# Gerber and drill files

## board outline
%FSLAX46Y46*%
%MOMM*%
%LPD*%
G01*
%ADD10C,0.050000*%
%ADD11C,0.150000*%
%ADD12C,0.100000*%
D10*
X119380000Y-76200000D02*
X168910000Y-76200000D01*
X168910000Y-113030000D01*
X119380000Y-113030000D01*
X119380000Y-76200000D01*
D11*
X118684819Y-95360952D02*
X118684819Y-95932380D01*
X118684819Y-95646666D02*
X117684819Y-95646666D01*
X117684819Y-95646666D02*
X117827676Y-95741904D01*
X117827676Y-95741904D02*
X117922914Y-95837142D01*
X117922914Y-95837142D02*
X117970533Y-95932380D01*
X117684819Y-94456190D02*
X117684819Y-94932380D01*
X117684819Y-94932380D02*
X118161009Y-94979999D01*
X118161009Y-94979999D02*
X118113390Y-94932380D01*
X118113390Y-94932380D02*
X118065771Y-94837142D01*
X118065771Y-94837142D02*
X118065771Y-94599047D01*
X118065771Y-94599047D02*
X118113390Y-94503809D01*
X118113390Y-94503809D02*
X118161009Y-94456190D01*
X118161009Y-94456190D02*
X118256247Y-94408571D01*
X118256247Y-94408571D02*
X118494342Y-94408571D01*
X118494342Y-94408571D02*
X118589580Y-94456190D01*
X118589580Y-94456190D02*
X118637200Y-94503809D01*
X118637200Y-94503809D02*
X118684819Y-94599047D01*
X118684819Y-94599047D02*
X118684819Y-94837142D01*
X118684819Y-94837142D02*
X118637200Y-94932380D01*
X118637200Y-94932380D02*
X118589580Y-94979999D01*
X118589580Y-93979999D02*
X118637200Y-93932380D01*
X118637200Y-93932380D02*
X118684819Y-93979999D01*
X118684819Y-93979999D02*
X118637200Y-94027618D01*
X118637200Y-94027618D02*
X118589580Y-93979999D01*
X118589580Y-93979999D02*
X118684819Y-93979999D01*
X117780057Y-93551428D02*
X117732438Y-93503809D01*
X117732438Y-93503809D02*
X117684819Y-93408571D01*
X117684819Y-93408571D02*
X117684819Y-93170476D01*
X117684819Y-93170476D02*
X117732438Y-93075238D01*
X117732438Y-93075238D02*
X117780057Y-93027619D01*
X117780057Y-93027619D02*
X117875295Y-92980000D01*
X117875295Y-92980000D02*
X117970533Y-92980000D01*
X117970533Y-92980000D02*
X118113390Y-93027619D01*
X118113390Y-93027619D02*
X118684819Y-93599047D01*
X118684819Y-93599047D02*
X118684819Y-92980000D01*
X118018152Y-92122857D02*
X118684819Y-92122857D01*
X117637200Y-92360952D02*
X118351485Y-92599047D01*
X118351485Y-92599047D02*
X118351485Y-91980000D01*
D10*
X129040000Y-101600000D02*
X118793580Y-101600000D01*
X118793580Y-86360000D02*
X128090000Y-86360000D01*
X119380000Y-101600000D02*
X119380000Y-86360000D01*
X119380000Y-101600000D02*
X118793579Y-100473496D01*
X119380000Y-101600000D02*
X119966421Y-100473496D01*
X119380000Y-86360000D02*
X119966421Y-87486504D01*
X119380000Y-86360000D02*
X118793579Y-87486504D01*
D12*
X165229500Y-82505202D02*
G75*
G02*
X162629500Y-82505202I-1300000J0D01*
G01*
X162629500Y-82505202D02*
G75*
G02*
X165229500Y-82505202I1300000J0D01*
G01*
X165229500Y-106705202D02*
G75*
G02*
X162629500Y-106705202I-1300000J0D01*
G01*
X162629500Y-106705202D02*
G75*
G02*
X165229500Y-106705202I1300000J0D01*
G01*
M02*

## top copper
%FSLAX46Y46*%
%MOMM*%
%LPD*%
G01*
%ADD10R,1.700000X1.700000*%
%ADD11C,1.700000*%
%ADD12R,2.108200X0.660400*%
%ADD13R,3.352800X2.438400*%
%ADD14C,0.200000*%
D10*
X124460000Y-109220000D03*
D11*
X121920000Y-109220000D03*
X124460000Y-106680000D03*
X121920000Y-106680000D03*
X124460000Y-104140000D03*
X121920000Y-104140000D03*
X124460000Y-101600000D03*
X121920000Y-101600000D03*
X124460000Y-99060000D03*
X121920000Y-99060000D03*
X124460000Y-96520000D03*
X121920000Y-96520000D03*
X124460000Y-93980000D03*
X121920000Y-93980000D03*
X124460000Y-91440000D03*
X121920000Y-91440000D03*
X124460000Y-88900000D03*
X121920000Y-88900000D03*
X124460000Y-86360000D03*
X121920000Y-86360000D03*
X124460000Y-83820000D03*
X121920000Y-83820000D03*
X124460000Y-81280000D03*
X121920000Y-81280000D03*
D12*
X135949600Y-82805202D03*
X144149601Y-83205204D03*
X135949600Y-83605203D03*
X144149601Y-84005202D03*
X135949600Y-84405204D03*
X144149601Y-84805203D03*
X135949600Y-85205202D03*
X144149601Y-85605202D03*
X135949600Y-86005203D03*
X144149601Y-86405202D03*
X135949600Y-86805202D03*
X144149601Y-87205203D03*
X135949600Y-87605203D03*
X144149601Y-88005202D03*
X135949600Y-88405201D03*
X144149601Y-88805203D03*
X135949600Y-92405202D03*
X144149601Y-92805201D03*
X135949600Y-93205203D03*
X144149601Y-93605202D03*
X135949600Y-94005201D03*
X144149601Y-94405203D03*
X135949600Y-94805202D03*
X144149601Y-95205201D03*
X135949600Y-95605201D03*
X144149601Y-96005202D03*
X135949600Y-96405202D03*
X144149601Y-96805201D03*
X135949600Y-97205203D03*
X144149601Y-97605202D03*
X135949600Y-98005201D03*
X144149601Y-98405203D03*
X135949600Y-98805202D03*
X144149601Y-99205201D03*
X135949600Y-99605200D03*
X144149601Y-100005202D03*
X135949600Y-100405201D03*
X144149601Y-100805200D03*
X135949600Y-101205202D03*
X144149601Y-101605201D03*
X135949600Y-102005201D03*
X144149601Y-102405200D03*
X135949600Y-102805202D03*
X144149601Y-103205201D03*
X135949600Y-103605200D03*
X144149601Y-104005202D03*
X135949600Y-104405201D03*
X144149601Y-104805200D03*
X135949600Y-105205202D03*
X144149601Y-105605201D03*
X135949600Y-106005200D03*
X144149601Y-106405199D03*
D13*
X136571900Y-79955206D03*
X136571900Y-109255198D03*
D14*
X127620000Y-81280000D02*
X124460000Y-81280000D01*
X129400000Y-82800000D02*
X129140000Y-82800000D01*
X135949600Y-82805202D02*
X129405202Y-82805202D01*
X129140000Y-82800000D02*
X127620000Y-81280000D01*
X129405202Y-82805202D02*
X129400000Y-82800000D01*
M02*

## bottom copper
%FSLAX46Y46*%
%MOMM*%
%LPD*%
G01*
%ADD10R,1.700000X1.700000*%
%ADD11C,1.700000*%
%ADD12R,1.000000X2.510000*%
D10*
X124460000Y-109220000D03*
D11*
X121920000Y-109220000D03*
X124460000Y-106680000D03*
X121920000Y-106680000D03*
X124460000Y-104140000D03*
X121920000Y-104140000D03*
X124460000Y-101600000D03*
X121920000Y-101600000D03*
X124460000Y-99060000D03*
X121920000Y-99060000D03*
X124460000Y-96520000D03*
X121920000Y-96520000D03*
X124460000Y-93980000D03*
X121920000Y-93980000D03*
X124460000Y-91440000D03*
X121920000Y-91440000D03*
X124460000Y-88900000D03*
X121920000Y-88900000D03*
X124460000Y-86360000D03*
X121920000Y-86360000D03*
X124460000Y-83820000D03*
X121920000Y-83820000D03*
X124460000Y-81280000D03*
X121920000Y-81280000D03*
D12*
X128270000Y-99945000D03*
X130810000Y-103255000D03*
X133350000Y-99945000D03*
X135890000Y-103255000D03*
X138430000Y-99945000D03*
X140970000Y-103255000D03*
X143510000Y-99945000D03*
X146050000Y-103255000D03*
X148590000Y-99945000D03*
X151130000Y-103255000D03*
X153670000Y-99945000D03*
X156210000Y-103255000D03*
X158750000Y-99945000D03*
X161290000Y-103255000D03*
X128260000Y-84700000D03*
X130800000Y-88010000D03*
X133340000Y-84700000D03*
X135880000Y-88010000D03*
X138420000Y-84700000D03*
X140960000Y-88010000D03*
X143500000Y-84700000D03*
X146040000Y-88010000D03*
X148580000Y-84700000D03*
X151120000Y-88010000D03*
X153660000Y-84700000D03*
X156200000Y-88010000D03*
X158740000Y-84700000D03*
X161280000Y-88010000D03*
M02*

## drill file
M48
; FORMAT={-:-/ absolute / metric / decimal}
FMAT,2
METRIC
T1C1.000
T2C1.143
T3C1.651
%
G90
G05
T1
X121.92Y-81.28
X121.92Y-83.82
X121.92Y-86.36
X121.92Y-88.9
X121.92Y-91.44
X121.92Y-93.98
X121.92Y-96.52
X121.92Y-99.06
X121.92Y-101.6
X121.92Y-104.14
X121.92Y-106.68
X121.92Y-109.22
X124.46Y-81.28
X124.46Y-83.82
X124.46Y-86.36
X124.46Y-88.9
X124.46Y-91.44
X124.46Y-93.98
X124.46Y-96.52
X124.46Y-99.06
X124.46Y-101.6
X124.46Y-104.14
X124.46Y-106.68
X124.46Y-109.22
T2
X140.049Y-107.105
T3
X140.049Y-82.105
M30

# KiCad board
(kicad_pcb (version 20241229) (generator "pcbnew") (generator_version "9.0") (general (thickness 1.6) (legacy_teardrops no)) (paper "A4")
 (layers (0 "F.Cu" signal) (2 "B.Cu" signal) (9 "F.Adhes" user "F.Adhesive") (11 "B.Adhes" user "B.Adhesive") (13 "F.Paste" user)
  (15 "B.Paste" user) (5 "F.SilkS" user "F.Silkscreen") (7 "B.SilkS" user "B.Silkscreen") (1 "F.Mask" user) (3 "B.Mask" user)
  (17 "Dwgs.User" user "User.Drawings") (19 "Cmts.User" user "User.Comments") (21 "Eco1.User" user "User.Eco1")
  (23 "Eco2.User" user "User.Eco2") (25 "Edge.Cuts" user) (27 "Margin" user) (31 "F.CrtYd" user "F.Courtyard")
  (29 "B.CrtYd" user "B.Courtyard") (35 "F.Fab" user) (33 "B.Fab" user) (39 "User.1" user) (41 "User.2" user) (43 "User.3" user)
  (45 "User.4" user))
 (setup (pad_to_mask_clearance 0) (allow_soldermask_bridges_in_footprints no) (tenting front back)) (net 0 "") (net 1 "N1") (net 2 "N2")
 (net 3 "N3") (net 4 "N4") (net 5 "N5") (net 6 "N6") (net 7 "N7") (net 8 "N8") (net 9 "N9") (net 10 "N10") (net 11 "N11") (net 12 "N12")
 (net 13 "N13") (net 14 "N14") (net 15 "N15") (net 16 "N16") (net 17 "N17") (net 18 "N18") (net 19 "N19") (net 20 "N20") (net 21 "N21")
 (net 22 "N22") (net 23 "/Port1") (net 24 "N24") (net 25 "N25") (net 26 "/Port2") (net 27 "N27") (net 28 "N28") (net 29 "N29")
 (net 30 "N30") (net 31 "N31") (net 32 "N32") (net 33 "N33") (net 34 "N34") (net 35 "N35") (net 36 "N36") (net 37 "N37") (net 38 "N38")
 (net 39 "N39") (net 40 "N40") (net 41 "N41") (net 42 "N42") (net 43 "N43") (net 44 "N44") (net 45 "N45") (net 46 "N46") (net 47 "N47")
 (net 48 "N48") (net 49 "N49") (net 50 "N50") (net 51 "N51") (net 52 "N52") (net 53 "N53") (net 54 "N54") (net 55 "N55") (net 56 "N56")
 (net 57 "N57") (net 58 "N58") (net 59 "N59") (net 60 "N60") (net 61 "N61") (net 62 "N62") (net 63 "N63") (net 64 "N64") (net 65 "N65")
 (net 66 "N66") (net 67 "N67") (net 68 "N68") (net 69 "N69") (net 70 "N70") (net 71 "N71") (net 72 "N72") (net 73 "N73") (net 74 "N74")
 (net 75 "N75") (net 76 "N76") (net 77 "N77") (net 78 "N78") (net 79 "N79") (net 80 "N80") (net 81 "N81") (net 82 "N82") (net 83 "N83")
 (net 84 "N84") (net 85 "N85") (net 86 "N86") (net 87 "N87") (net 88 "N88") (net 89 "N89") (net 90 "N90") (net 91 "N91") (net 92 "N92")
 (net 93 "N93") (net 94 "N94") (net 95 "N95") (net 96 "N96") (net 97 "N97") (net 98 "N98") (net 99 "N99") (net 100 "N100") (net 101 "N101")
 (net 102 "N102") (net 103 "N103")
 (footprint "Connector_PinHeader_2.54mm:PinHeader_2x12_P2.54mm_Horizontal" (layer "F.Cu") (at 124.46 109.22 180)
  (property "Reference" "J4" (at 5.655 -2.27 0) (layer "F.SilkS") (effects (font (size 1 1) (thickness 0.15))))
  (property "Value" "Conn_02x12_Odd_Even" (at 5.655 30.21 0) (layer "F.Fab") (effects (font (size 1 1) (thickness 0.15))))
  (pad "1" thru_hole rect (at 0 0 180) (size 1.7 1.7) (drill 1) (layers "*.Cu" "*.Mask") (remove_unused_layers no) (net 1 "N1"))
  (pad "2" thru_hole circle (at 2.54 0 180) (size 1.7 1.7) (drill 1) (layers "*.Cu" "*.Mask") (remove_unused_layers no) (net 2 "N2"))
  (pad "3" thru_hole circle (at 0 2.54 180) (size 1.7 1.7) (drill 1) (layers "*.Cu" "*.Mask") (remove_unused_layers no) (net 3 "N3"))
  (pad "4" thru_hole circle (at 2.54 2.54 180) (size 1.7 1.7) (drill 1) (layers "*.Cu" "*.Mask") (remove_unused_layers no) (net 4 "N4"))
  (pad "5" thru_hole circle (at 0 5.08 180) (size 1.7 1.7) (drill 1) (layers "*.Cu" "*.Mask") (remove_unused_layers no) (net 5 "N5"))
  (pad "6" thru_hole circle (at 2.54 5.08 180) (size 1.7 1.7) (drill 1) (layers "*.Cu" "*.Mask") (remove_unused_layers no) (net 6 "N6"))
  (pad "7" thru_hole circle (at 0 7.62 180) (size 1.7 1.7) (drill 1) (layers "*.Cu" "*.Mask") (remove_unused_layers no) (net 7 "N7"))
  (pad "8" thru_hole circle (at 2.54 7.62 180) (size 1.7 1.7) (drill 1) (layers "*.Cu" "*.Mask") (remove_unused_layers no) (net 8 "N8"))
  (pad "9" thru_hole circle (at 0 10.16 180) (size 1.7 1.7) (drill 1) (layers "*.Cu" "*.Mask") (remove_unused_layers no) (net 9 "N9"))
  (pad "10" thru_hole circle (at 2.54 10.16 180) (size 1.7 1.7) (drill 1) (layers "*.Cu" "*.Mask") (remove_unused_layers no) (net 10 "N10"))
  (pad "11" thru_hole circle (at 0 12.7 180) (size 1.7 1.7) (drill 1) (layers "*.Cu" "*.Mask") (remove_unused_layers no) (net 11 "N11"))
  (pad "12" thru_hole circle (at 2.54 12.7 180) (size 1.7 1.7) (drill 1) (layers "*.Cu" "*.Mask") (remove_unused_layers no) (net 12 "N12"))
  (pad "13" thru_hole circle (at 0 15.24 180) (size 1.7 1.7) (drill 1) (layers "*.Cu" "*.Mask") (remove_unused_layers no) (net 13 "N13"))
  (pad "14" thru_hole circle (at 2.54 15.24 180) (size 1.7 1.7) (drill 1) (layers "*.Cu" "*.Mask") (remove_unused_layers no) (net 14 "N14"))
  (pad "15" thru_hole circle (at 0 17.78 180) (size 1.7 1.7) (drill 1) (layers "*.Cu" "*.Mask") (remove_unused_layers no) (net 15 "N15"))
  (pad "16" thru_hole circle (at 2.54 17.78 180) (size 1.7 1.7) (drill 1) (layers "*.Cu" "*.Mask") (remove_unused_layers no) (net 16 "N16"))
  (pad "17" thru_hole circle (at 0 20.32 180) (size 1.7 1.7) (drill 1) (layers "*.Cu" "*.Mask") (remove_unused_layers no) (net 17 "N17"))
  (pad "18" thru_hole circle (at 2.54 20.32 180) (size 1.7 1.7) (drill 1) (layers "*.Cu" "*.Mask") (remove_unused_layers no) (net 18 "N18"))
  (pad "19" thru_hole circle (at 0 22.86 180) (size 1.7 1.7) (drill 1) (layers "*.Cu" "*.Mask") (remove_unused_layers no) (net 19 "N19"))
  (pad "20" thru_hole circle (at 2.54 22.86 180) (size 1.7 1.7) (drill 1) (layers "*.Cu" "*.Mask") (remove_unused_layers no) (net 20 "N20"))
  (pad "21" thru_hole circle (at 0 25.4 180) (size 1.7 1.7) (drill 1) (layers "*.Cu" "*.Mask") (remove_unused_layers no) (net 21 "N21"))
  (pad "22" thru_hole circle (at 2.54 25.4 180) (size 1.7 1.7) (drill 1) (layers "*.Cu" "*.Mask") (remove_unused_layers no) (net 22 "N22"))
  (pad "23" thru_hole circle (at 0 27.94 180) (size 1.7 1.7) (drill 1) (layers "*.Cu" "*.Mask") (remove_unused_layers no) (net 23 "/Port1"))
  (pad "24" thru_hole circle (at 2.54 27.94 180) (size 1.7 1.7) (drill 1) (layers "*.Cu" "*.Mask") (remove_unused_layers no) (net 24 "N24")))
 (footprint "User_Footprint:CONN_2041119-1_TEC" (layer "F.Cu") (at 140.0495 94.605202 -90)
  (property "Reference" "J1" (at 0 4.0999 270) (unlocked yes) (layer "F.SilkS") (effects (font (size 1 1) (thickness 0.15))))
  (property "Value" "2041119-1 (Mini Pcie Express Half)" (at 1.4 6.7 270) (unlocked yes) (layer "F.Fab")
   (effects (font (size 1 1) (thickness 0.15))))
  (fp_circle (center -12.1 -23.88) (end -10.8 -23.88) (stroke (width 0.1) (type solid)) (fill no) (layer "Edge.Cuts"))
  (fp_circle (center 12.1 -23.88) (end 13.4 -23.88) (stroke (width 0.1) (type solid)) (fill no) (layer "Edge.Cuts"))
  (pad "" np_thru_hole circle (at -12.500102 0 270) (size 1.651 1.651) (drill 1.651) (layers))
  (pad "" np_thru_hole circle (at 12.500102 0 270) (size 1.143 1.143) (drill 1.143) (layers))
  (pad "1" smd rect (at -11.8 4.0999 270) (size 0.6604 2.1082) (layers "F.Cu" "F.Mask" "F.Paste") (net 23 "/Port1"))
  (pad "2" smd rect (at -11.399998 -4.100101 270) (size 0.6604 2.1082) (layers "F.Cu" "F.Mask" "F.Paste") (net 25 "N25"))
  (pad "3" smd rect (at -10.999999 4.0999 270) (size 0.6604 2.1082) (layers "F.Cu" "F.Mask" "F.Paste") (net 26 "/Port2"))
  (pad "4" smd rect (at -10.6 -4.100101 270) (size 0.6604 2.1082) (layers "F.Cu" "F.Mask" "F.Paste") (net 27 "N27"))
  (pad "5" smd rect (at -10.199998 4.0999 270) (size 0.6604 2.1082) (layers "F.Cu" "F.Mask" "F.Paste") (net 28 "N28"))
  (pad "6" smd rect (at -9.799999 -4.100101 270) (size 0.6604 2.1082) (layers "F.Cu" "F.Mask" "F.Paste") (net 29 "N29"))
  (pad "7" smd rect (at -9.4 4.0999 270) (size 0.6604 2.1082) (layers "F.Cu" "F.Mask" "F.Paste") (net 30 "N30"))
  (pad "8" smd rect (at -9 -4.100101 270) (size 0.6604 2.1082) (layers "F.Cu" "F.Mask" "F.Paste") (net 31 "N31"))
  (pad "9" smd rect (at -8.599999 4.0999 270) (size 0.6604 2.1082) (layers "F.Cu" "F.Mask" "F.Paste") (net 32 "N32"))
  (pad "10" smd rect (at -8.2 -4.100101 270) (size 0.6604 2.1082) (layers "F.Cu" "F.Mask" "F.Paste") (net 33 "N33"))
  (pad "11" smd rect (at -7.8 4.0999 270) (size 0.6604 2.1082) (layers "F.Cu" "F.Mask" "F.Paste") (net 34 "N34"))
  (pad "12" smd rect (at -7.399999 -4.100101 270) (size 0.6604 2.1082) (layers "F.Cu" "F.Mask" "F.Paste") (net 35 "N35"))
  (pad "13" smd rect (at -6.999999 4.0999 270) (size 0.6604 2.1082) (layers "F.Cu" "F.Mask" "F.Paste") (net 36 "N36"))
  (pad "14" smd rect (at -6.6 -4.100101 270) (size 0.6604 2.1082) (layers "F.Cu" "F.Mask" "F.Paste") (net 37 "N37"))
  (pad "15" smd rect (at -6.200001 4.0999 270) (size 0.6604 2.1082) (layers "F.Cu" "F.Mask" "F.Paste") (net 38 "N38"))
  (pad "16" smd rect (at -5.799999 -4.100101 270) (size 0.6604 2.1082) (layers "F.Cu" "F.Mask" "F.Paste") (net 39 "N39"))
  (pad "17" smd rect (at -2.2 4.0999 270) (size 0.6604 2.1082) (layers "F.Cu" "F.Mask" "F.Paste") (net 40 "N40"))
  (pad "18" smd rect (at -1.800001 -4.100101 270) (size 0.6604 2.1082) (layers "F.Cu" "F.Mask" "F.Paste") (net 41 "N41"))
  (pad "19" smd rect (at -1.399999 4.0999 270) (size 0.6604 2.1082) (layers "F.Cu" "F.Mask" "F.Paste") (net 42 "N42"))
  (pad "20" smd rect (at -1 -4.100101 270) (size 0.6604 2.1082) (layers "F.Cu" "F.Mask" "F.Paste") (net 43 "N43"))
  (pad "21" smd rect (at -0.600001 4.0999 270) (size 0.6604 2.1082) (layers "F.Cu" "F.Mask" "F.Paste") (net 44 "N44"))
  (pad "22" smd rect (at -0.199999 -4.100101 270) (size 0.6604 2.1082) (layers "F.Cu" "F.Mask" "F.Paste") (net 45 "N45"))
  (pad "23" smd rect (at 0.2 4.0999 270) (size 0.6604 2.1082) (layers "F.Cu" "F.Mask" "F.Paste") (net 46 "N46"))
  (pad "24" smd rect (at 0.599999 -4.100101 270) (size 0.6604 2.1082) (layers "F.Cu" "F.Mask" "F.Paste") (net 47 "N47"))
  (pad "25" smd rect (at 0.999999 4.0999 270) (size 0.6604 2.1082) (layers "F.Cu" "F.Mask" "F.Paste") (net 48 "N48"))
  (pad "26" smd rect (at 1.4 -4.100101 270) (size 0.6604 2.1082) (layers "F.Cu" "F.Mask" "F.Paste") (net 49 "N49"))
  (pad "27" smd rect (at 1.8 4.0999 270) (size 0.6604 2.1082) (layers "F.Cu" "F.Mask" "F.Paste") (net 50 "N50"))
  (pad "28" smd rect (at 2.199999 -4.100101 270) (size 0.6604 2.1082) (layers "F.Cu" "F.Mask" "F.Paste") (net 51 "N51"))
  (pad "29" smd rect (at 2.600001 4.0999 270) (size 0.6604 2.1082) (layers "F.Cu" "F.Mask" "F.Paste") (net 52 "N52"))
  (pad "30" smd rect (at 3 -4.100101 270) (size 0.6604 2.1082) (layers "F.Cu" "F.Mask" "F.Paste") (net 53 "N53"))
  (pad "31" smd rect (at 3.399999 4.0999 270) (size 0.6604 2.1082) (layers "F.Cu" "F.Mask" "F.Paste") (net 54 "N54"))
  (pad "32" smd rect (at 3.800001 -4.100101 270) (size 0.6604 2.1082) (layers "F.Cu" "F.Mask" "F.Paste") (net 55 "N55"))
  (pad "33" smd rect (at 4.2 4.0999 270) (size 0.6604 2.1082) (layers "F.Cu" "F.Mask" "F.Paste") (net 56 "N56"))
  (pad "34" smd rect (at 4.599999 -4.100101 270) (size 0.6604 2.1082) (layers "F.Cu" "F.Mask" "F.Paste") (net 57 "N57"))
  (pad "35" smd rect (at 4.999998 4.0999 270) (size 0.6604 2.1082) (layers "F.Cu" "F.Mask" "F.Paste") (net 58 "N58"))
  (pad "36" smd rect (at 5.4 -4.100101 270) (size 0.6604 2.1082) (layers "F.Cu" "F.Mask" "F.Paste") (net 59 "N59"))
  (pad "37" smd rect (at 5.799999 4.0999 270) (size 0.6604 2.1082) (layers "F.Cu" "F.Mask" "F.Paste") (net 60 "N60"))
  (pad "38" smd rect (at 6.199998 -4.100101 270) (size 0.6604 2.1082) (layers "F.Cu" "F.Mask" "F.Paste") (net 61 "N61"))
  (pad "39" smd rect (at 6.6 4.0999 270) (size 0.6604 2.1082) (layers "F.Cu" "F.Mask" "F.Paste") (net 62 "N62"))
  (pad "40" smd rect (at 6.999999 -4.100101 270) (size 0.6604 2.1082) (layers "F.Cu" "F.Mask" "F.Paste") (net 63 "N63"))
  (pad "41" smd rect (at 7.399999 4.0999 270) (size 0.6604 2.1082) (layers "F.Cu" "F.Mask" "F.Paste") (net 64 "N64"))
  (pad "42" smd rect (at 7.799998 -4.100101 270) (size 0.6604 2.1082) (layers "F.Cu" "F.Mask" "F.Paste") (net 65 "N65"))
  (pad "43" smd rect (at 8.2 4.0999 270) (size 0.6604 2.1082) (layers "F.Cu" "F.Mask" "F.Paste") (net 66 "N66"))
  (pad "44" smd rect (at 8.599999 -4.100101 270) (size 0.6604 2.1082) (layers "F.Cu" "F.Mask" "F.Paste") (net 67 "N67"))
  (pad "45" smd rect (at 8.999998 4.0999 270) (size 0.6604 2.1082) (layers "F.Cu" "F.Mask" "F.Paste") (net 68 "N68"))
  (pad "46" smd rect (at 9.4 -4.100101 270) (size 0.6604 2.1082) (layers "F.Cu" "F.Mask" "F.Paste") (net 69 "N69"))
  (pad "47" smd rect (at 9.799999 4.0999 270) (size 0.6604 2.1082) (layers "F.Cu" "F.Mask" "F.Paste") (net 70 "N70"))
  (pad "48" smd rect (at 10.199998 -4.100101 270) (size 0.6604 2.1082) (layers "F.Cu" "F.Mask" "F.Paste") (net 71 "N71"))
  (pad "49" smd rect (at 10.6 4.0999 270) (size 0.6604 2.1082) (layers "F.Cu" "F.Mask" "F.Paste") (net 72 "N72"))
  (pad "50" smd rect (at 10.999999 -4.100101 270) (size 0.6604 2.1082) (layers "F.Cu" "F.Mask" "F.Paste") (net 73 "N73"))
  (pad "51" smd rect (at 11.399998 4.0999 270) (size 0.6604 2.1082) (layers "F.Cu" "F.Mask" "F.Paste") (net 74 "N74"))
  (pad "52" smd rect (at 11.799997 -4.100101 270) (size 0.6604 2.1082) (layers "F.Cu" "F.Mask" "F.Paste") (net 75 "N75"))
  (pad "53" smd rect (at -14.649996 3.4776) (size 3.3528 2.4384) (layers "F.Cu" "F.Mask" "F.Paste"))
  (pad "54" smd rect (at 14.649996 3.4776) (size 3.3528 2.4384) (layers "F.Cu" "F.Mask" "F.Paste")))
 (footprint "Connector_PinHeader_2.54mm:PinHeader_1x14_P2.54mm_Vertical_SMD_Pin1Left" (layer "B.Cu") (at 144.78 101.6 -90)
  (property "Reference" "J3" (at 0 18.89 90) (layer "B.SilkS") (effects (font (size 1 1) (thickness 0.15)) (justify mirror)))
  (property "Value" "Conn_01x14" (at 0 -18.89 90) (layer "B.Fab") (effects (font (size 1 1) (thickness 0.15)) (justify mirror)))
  (pad "1" smd rect (at -1.655 16.51 270) (size 2.51 1) (layers "B.Cu" "B.Mask" "B.Paste") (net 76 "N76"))
  (pad "2" smd rect (at 1.655 13.97 270) (size 2.51 1) (layers "B.Cu" "B.Mask" "B.Paste") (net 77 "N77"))
  (pad "3" smd rect (at -1.655 11.43 270) (size 2.51 1) (layers "B.Cu" "B.Mask" "B.Paste") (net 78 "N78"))
  (pad "4" smd rect (at 1.655 8.89 270) (size 2.51 1) (layers "B.Cu" "B.Mask" "B.Paste") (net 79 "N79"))
  (pad "5" smd rect (at -1.655 6.35 270) (size 2.51 1) (layers "B.Cu" "B.Mask" "B.Paste") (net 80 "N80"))
  (pad "6" smd rect (at 1.655 3.81 270) (size 2.51 1) (layers "B.Cu" "B.Mask" "B.Paste") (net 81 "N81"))
  (pad "7" smd rect (at -1.655 1.27 270) (size 2.51 1) (layers "B.Cu" "B.Mask" "B.Paste") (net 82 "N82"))
  (pad "8" smd rect (at 1.655 -1.27 270) (size 2.51 1) (layers "B.Cu" "B.Mask" "B.Paste") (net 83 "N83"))
  (pad "9" smd rect (at -1.655 -3.81 270) (size 2.51 1) (layers "B.Cu" "B.Mask" "B.Paste") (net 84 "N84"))
  (pad "10" smd rect (at 1.655 -6.35 270) (size 2.51 1) (layers "B.Cu" "B.Mask" "B.Paste") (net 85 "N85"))
  (pad "11" smd rect (at -1.655 -8.89 270) (size 2.51 1) (layers "B.Cu" "B.Mask" "B.Paste") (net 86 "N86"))
  (pad "12" smd rect (at 1.655 -11.43 270) (size 2.51 1) (layers "B.Cu" "B.Mask" "B.Paste") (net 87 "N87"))
  (pad "13" smd rect (at -1.655 -13.97 270) (size 2.51 1) (layers "B.Cu" "B.Mask" "B.Paste") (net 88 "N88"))
  (pad "14" smd rect (at 1.655 -16.51 270) (size 2.51 1) (layers "B.Cu" "B.Mask" "B.Paste") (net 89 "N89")))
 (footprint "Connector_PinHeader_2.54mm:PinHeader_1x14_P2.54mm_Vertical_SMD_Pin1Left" (layer "B.Cu") (at 144.77 86.355 -90)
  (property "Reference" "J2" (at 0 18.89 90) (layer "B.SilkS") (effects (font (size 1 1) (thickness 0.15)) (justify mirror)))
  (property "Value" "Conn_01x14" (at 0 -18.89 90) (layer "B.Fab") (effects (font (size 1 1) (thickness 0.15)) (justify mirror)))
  (pad "1" smd rect (at -1.655 16.51 270) (size 2.51 1) (layers "B.Cu" "B.Mask" "B.Paste") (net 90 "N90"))
  (pad "2" smd rect (at 1.655 13.97 270) (size 2.51 1) (layers "B.Cu" "B.Mask" "B.Paste") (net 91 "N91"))
  (pad "3" smd rect (at -1.655 11.43 270) (size 2.51 1) (layers "B.Cu" "B.Mask" "B.Paste") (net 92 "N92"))
  (pad "4" smd rect (at 1.655 8.89 270) (size 2.51 1) (layers "B.Cu" "B.Mask" "B.Paste") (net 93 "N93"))
  (pad "5" smd rect (at -1.655 6.35 270) (size 2.51 1) (layers "B.Cu" "B.Mask" "B.Paste") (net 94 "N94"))
  (pad "6" smd rect (at 1.655 3.81 270) (size 2.51 1) (layers "B.Cu" "B.Mask" "B.Paste") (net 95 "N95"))
  (pad "7" smd rect (at -1.655 1.27 270) (size 2.51 1) (layers "B.Cu" "B.Mask" "B.Paste") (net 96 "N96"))
  (pad "8" smd rect (at 1.655 -1.27 270) (size 2.51 1) (layers "B.Cu" "B.Mask" "B.Paste") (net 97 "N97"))
  (pad "9" smd rect (at -1.655 -3.81 270) (size 2.51 1) (layers "B.Cu" "B.Mask" "B.Paste") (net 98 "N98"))
  (pad "10" smd rect (at 1.655 -6.35 270) (size 2.51 1) (layers "B.Cu" "B.Mask" "B.Paste") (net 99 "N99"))
  (pad "11" smd rect (at -1.655 -8.89 270) (size 2.51 1) (layers "B.Cu" "B.Mask" "B.Paste") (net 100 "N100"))
  (pad "12" smd rect (at 1.655 -11.43 270) (size 2.51 1) (layers "B.Cu" "B.Mask" "B.Paste") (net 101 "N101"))
  (pad "13" smd rect (at -1.655 -13.97 270) (size 2.51 1) (layers "B.Cu" "B.Mask" "B.Paste") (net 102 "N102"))
  (pad "14" smd rect (at 1.655 -16.51 270) (size 2.51 1) (layers "B.Cu" "B.Mask" "B.Paste") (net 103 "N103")))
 (gr_rect (start 119.38 76.2) (end 168.91 113.03) (stroke (width 0.05) (type default)) (fill no) (layer "Edge.Cuts"))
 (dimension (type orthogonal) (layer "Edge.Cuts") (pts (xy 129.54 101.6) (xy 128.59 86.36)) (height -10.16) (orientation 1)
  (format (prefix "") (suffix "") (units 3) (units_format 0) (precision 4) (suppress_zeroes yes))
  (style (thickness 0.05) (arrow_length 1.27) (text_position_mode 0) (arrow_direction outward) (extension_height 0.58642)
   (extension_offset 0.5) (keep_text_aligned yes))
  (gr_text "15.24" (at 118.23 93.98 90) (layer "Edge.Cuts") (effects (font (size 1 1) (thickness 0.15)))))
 (segment (start 127.62 81.28) (end 124.46 81.28) (width 0.2) (layer "F.Cu") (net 23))
 (segment (start 129.4 82.8) (end 129.14 82.8) (width 0.2) (layer "F.Cu") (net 23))
 (segment (start 135.9496 82.805202) (end 129.405202 82.805202) (width 0.2) (layer "F.Cu") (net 23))
 (segment (start 129.14 82.8) (end 127.62 81.28) (width 0.2) (layer "F.Cu") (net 23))
 (segment (start 129.405202 82.805202) (end 129.4 82.8) (width 0.2) (layer "F.Cu") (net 23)))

